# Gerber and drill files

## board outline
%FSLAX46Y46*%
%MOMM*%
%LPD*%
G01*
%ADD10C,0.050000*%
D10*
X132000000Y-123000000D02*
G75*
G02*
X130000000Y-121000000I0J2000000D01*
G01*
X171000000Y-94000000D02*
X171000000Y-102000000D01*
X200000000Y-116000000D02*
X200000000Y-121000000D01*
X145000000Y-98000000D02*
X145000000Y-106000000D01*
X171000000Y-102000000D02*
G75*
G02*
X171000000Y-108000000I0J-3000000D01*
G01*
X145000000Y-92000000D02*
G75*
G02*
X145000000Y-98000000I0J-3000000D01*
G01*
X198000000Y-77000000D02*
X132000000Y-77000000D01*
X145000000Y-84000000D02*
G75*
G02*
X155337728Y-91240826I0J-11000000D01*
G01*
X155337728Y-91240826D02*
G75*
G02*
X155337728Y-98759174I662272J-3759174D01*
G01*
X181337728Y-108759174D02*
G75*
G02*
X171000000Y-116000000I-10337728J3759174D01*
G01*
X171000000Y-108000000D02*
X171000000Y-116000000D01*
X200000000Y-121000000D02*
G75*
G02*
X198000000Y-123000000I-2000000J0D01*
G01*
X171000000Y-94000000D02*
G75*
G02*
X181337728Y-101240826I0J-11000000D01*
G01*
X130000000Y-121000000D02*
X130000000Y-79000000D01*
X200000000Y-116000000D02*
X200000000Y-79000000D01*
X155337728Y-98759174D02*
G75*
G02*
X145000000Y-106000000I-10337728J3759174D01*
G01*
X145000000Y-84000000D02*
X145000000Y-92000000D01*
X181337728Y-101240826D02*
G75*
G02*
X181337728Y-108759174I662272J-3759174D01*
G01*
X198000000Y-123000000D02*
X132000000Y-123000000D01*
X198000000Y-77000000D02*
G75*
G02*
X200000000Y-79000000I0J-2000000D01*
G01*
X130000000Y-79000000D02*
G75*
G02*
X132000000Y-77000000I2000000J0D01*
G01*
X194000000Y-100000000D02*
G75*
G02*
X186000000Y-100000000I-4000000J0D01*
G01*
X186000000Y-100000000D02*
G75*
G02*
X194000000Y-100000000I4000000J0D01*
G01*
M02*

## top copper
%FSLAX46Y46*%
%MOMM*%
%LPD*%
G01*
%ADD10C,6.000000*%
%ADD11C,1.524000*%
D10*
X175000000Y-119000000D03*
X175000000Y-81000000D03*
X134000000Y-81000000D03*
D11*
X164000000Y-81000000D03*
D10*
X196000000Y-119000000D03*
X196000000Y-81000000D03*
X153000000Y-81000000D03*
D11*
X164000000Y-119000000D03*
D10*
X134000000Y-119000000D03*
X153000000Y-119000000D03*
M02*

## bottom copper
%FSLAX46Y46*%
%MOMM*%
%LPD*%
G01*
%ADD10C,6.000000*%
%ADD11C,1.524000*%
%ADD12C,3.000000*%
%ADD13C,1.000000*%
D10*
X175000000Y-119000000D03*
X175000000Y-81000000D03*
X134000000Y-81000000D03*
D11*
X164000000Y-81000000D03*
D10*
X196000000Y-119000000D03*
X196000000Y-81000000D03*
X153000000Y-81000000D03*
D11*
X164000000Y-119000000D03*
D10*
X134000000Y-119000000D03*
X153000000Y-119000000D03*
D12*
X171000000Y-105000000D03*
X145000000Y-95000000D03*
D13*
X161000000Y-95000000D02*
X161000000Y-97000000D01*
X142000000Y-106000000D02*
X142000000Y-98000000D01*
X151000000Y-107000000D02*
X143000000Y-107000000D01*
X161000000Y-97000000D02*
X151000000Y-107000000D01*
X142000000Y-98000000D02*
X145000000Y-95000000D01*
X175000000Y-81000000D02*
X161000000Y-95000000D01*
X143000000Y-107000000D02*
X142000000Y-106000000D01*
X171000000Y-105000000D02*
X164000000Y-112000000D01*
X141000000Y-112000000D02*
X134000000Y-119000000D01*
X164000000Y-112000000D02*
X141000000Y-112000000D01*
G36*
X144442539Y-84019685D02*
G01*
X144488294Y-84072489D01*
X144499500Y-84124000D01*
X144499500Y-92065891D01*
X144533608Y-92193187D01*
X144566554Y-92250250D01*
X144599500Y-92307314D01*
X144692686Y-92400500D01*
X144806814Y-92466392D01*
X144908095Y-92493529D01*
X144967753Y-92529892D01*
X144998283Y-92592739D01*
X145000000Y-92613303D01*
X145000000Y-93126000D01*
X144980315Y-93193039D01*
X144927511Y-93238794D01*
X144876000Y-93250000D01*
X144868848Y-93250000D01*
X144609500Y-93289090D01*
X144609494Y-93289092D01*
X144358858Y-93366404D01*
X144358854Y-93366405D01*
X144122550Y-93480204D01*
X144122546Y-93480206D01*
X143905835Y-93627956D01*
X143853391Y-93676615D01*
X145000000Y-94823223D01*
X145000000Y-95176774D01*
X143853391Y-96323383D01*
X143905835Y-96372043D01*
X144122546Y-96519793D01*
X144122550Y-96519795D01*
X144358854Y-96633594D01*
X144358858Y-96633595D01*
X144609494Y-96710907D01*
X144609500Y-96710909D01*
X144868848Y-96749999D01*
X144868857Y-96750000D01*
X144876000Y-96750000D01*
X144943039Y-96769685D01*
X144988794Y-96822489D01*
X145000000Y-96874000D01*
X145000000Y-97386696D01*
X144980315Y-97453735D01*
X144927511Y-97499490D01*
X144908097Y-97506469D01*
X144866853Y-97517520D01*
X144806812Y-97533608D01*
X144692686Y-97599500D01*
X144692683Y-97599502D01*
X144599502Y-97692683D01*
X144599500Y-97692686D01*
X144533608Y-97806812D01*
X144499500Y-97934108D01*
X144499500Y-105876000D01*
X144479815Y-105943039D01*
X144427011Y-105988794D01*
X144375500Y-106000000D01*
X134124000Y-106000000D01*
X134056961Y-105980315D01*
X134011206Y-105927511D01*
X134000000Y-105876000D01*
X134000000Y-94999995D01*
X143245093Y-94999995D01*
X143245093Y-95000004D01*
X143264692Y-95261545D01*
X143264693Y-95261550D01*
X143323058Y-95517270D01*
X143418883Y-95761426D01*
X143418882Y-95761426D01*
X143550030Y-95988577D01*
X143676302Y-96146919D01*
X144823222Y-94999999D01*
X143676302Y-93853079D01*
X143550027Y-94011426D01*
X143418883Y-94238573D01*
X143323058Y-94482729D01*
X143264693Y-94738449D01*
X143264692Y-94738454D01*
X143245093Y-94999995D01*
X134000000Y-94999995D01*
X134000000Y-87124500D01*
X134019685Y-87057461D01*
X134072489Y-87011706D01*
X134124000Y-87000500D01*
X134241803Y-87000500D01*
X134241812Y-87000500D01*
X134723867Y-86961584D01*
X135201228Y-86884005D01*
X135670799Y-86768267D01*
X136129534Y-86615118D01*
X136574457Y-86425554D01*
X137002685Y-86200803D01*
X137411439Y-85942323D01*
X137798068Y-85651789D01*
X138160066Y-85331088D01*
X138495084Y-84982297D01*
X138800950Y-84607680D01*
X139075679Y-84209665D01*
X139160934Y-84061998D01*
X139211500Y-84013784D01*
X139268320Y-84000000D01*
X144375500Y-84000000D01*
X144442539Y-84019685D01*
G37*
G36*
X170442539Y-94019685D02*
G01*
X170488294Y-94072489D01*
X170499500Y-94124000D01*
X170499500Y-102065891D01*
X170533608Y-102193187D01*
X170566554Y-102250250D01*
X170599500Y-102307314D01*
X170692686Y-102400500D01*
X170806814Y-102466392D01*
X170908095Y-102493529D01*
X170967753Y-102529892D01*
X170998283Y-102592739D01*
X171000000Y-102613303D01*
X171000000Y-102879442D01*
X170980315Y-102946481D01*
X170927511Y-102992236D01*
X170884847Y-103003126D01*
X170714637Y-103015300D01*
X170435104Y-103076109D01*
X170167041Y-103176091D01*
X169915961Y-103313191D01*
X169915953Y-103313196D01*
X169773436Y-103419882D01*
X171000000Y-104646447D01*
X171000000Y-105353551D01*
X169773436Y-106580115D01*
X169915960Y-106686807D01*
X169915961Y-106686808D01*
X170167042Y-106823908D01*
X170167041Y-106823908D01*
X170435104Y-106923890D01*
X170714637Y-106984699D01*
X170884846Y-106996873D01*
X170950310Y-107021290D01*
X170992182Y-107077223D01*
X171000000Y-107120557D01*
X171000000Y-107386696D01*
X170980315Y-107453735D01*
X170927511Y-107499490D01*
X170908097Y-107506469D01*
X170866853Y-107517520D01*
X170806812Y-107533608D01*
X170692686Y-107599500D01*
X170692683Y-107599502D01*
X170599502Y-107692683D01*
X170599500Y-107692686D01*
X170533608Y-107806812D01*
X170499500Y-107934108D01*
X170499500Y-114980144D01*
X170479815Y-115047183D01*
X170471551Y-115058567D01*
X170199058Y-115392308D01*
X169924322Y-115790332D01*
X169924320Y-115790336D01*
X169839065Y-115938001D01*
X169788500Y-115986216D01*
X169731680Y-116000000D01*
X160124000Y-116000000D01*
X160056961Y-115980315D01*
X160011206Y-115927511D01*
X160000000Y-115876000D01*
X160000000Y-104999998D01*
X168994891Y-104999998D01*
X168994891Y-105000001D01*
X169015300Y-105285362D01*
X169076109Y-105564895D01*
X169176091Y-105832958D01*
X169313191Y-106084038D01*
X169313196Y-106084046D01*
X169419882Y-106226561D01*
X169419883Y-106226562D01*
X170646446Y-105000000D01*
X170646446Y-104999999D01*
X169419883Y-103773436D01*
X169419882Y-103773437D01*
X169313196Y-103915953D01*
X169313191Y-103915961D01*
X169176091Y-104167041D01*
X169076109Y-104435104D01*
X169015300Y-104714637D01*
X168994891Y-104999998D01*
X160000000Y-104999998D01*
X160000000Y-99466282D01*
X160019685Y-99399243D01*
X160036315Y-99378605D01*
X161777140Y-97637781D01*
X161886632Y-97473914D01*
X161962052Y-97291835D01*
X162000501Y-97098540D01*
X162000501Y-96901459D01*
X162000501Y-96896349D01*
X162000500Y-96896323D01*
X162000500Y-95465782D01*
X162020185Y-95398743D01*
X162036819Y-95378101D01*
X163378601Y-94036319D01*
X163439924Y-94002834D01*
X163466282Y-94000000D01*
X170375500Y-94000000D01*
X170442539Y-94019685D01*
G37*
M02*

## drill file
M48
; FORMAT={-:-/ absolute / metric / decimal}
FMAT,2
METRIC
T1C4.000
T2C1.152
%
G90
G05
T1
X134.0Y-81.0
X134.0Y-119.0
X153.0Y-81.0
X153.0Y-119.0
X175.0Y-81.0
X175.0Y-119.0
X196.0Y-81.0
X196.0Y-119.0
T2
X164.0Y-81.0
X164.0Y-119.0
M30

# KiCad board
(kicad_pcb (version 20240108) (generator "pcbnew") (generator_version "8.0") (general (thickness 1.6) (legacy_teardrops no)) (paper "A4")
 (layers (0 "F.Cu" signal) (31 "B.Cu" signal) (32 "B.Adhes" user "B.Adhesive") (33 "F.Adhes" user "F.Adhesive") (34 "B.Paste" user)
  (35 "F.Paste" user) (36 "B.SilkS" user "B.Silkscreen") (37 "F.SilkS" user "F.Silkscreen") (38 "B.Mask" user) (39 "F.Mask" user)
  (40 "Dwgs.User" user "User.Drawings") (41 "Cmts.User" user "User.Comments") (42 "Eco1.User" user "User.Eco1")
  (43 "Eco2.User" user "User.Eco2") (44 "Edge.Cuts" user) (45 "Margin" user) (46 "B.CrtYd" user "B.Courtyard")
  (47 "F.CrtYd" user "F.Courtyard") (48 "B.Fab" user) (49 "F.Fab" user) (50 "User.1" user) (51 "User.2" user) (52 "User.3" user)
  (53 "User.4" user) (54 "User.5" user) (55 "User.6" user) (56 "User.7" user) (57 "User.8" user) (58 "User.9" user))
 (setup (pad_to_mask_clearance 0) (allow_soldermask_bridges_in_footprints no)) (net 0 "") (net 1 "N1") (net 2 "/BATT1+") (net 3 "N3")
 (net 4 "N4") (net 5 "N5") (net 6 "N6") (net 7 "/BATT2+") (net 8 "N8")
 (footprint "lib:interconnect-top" (layer "F.Cu") (at 175 119)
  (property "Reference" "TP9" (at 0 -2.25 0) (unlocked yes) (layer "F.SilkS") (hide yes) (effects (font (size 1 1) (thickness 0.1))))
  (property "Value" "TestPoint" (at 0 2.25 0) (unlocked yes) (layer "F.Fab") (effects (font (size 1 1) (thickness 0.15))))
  (pad "1" thru_hole circle (at 0 0) (size 6 6) (drill 4) (layers "*.Cu" "*.Mask") (remove_unused_layers no) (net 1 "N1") (clearance 3)))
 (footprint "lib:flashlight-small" (layer "F.Cu") (at 193 110 0.13)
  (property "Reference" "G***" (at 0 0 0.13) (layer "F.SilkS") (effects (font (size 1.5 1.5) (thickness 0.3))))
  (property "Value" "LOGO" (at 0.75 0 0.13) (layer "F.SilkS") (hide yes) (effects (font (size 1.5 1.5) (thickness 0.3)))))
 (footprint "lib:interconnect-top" (layer "F.Cu") (at 175 81)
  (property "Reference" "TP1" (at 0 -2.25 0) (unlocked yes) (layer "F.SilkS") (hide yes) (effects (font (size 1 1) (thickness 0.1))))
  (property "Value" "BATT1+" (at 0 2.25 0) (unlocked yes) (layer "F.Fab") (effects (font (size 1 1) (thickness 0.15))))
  (pad "1" thru_hole circle (at 0 0) (size 6 6) (drill 4) (layers "*.Cu" "*.Mask") (remove_unused_layers no) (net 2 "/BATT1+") (clearance 3)))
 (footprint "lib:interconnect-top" (layer "F.Cu") (at 134 81)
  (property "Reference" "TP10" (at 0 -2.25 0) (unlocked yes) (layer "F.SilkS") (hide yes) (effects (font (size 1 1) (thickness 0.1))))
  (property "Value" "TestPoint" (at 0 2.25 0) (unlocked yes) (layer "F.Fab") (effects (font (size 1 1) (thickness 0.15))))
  (pad "1" thru_hole circle (at 0 0) (size 6 6) (drill 4) (layers "*.Cu" "*.Mask") (remove_unused_layers no) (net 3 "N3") (clearance 3)))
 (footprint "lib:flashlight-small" (layer "F.Cu") (at 193 90 0.13)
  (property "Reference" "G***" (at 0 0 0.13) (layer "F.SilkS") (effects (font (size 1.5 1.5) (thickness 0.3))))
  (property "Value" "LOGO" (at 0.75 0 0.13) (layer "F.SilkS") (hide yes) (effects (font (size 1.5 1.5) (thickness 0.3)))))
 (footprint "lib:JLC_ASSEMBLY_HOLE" (layer "F.Cu") (at 164 81)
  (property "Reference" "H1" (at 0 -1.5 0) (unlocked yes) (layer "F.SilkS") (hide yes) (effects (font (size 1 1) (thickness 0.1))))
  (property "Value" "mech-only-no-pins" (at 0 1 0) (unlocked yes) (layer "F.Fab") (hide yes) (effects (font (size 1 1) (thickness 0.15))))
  (pad "" np_thru_hole circle (at 0 0) (size 1.524 1.524) (drill 1.152) (layers "F&B.Cu" "*.Mask")))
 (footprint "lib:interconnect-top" (layer "F.Cu") (at 196 119)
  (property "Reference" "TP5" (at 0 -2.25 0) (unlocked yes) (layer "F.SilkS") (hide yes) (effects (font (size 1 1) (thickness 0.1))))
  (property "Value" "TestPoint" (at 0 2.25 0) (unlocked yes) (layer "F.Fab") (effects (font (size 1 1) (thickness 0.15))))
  (pad "1" thru_hole circle (at 0 0) (size 6 6) (drill 4) (layers "*.Cu" "*.Mask") (remove_unused_layers no) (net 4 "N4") (clearance 3)))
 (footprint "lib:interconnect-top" (layer "F.Cu") (at 196 81)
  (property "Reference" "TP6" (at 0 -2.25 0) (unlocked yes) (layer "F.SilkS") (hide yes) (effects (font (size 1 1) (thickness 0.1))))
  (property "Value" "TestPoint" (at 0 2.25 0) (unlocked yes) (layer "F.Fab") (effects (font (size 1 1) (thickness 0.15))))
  (pad "1" thru_hole circle (at 0 0) (size 6 6) (drill 4) (layers "*.Cu" "*.Mask") (remove_unused_layers no) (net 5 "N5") (clearance 3)))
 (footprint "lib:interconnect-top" (layer "F.Cu") (at 153 81)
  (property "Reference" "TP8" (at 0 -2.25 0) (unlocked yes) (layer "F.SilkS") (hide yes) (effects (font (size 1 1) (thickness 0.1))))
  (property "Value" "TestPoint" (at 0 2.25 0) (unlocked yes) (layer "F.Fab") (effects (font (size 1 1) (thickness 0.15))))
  (pad "1" thru_hole circle (at 0 0) (size 6 6) (drill 4) (layers "*.Cu" "*.Mask") (remove_unused_layers no) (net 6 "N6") (clearance 3)))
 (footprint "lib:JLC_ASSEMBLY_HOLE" (layer "F.Cu") (at 164 119)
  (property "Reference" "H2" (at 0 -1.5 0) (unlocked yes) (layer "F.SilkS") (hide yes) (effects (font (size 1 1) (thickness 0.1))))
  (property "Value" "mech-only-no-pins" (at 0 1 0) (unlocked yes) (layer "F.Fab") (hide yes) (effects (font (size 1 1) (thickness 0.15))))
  (pad "" np_thru_hole circle (at 0 0) (size 1.524 1.524) (drill 1.152) (layers "F&B.Cu" "*.Mask")))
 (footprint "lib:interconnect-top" (layer "F.Cu") (at 134 119)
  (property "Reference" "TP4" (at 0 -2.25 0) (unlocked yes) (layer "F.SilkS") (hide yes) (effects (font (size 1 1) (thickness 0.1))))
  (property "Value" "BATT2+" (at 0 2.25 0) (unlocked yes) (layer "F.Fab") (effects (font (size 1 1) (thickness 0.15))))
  (pad "1" thru_hole circle (at 0 0) (size 6 6) (drill 4) (layers "*.Cu" "*.Mask") (remove_unused_layers no) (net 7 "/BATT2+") (clearance 3)))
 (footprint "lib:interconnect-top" (layer "F.Cu") (at 153 119)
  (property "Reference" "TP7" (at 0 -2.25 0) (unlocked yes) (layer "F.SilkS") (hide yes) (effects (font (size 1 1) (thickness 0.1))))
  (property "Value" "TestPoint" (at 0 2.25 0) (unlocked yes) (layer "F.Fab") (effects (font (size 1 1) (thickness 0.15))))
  (pad "1" thru_hole circle (at 0 0) (size 6 6) (drill 4) (layers "*.Cu" "*.Mask") (remove_unused_layers no) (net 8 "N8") (clearance 3)))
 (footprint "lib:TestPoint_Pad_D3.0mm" (layer "B.Cu") (at 171 105 180)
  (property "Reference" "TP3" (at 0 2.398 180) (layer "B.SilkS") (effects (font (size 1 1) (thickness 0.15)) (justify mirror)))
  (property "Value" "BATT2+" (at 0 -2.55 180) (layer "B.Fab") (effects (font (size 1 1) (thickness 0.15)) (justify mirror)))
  (pad "1" smd circle (at 0 0 180) (size 3 3) (layers "B.Cu" "B.Mask") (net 7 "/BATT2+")))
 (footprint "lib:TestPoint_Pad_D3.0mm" (layer "B.Cu") (at 145 95 180)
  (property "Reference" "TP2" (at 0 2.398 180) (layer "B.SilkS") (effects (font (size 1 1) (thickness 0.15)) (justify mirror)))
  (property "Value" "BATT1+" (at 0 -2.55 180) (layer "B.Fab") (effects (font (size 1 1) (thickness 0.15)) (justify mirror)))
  (pad "1" smd circle (at 0 0 180) (size 3 3) (layers "B.Cu" "B.Mask") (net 2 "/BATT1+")))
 (gr_arc (start 132 123) (mid 130.585786 122.414214) (end 130 121) (stroke (width 0.05) (type default)) (layer "Edge.Cuts"))
 (gr_line (start 171 94) (end 171 102) (stroke (width 0.05) (type default)) (layer "Edge.Cuts"))
 (gr_line (start 200 116) (end 200 121) (stroke (width 0.05) (type default)) (layer "Edge.Cuts"))
 (gr_line (start 145 98) (end 145 106) (stroke (width 0.05) (type default)) (layer "Edge.Cuts"))
 (gr_arc (start 171 102) (mid 174 105) (end 171 108) (stroke (width 0.05) (type default)) (layer "Edge.Cuts"))
 (gr_arc (start 145 92) (mid 148 95) (end 145 98) (stroke (width 0.05) (type default)) (layer "Edge.Cuts"))
 (gr_line (start 198 77) (end 132 77) (stroke (width 0.05) (type default)) (layer "Edge.Cuts"))
 (gr_arc (start 145 84) (mid 151.310669 85.990258) (end 155.337728 91.240826) (stroke (width 0.05) (type default)) (layer "Edge.Cuts"))
 (gr_arc (start 155.337728 91.240826) (mid 159.817066 95) (end 155.337728 98.759174) (stroke (width 0.05) (type default))
  (layer "Edge.Cuts"))
 (gr_arc (start 181.337728 108.759174) (mid 177.310669 114.009742) (end 171 116) (stroke (width 0.05) (type default)) (layer "Edge.Cuts"))
 (gr_line (start 171 108) (end 171 116) (stroke (width 0.05) (type default)) (layer "Edge.Cuts"))
 (gr_arc (start 200 121) (mid 199.414214 122.414214) (end 198 123) (stroke (width 0.05) (type default)) (layer "Edge.Cuts"))
 (gr_arc (start 171 94) (mid 177.310669 95.990258) (end 181.337728 101.240826) (stroke (width 0.05) (type default)) (layer "Edge.Cuts"))
 (gr_line (start 130 121) (end 130 79) (stroke (width 0.05) (type default)) (layer "Edge.Cuts"))
 (gr_line (start 200 116) (end 200 79) (stroke (width 0.05) (type default)) (layer "Edge.Cuts"))
 (gr_arc (start 155.337728 98.759174) (mid 151.310669 104.009742) (end 145 106) (stroke (width 0.05) (type default)) (layer "Edge.Cuts"))
 (gr_line (start 145 84) (end 145 92) (stroke (width 0.05) (type default)) (layer "Edge.Cuts"))
 (gr_arc (start 181.337728 101.240826) (mid 185.817066 105) (end 181.337728 108.759174) (stroke (width 0.05) (type default))
  (layer "Edge.Cuts"))
 (gr_line (start 198 123) (end 132 123) (stroke (width 0.05) (type default)) (layer "Edge.Cuts"))
 (gr_arc (start 198 77) (mid 199.414214 77.585786) (end 200 79) (stroke (width 0.05) (type default)) (layer "Edge.Cuts"))
 (gr_arc (start 130 79) (mid 130.585786 77.585786) (end 132 77) (stroke (width 0.05) (type default)) (layer "Edge.Cuts"))
 (gr_circle (center 190 100) (end 194 100) (stroke (width 0.05) (type default)) (fill none) (layer "Edge.Cuts"))
 (segment (start 161 95) (end 161 97) (width 1) (layer "B.Cu") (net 2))
 (segment (start 142 106) (end 142 98) (width 1) (layer "B.Cu") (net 2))
 (segment (start 151 107) (end 143 107) (width 1) (layer "B.Cu") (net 2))
 (segment (start 161 97) (end 151 107) (width 1) (layer "B.Cu") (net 2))
 (segment (start 142 98) (end 145 95) (width 1) (layer "B.Cu") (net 2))
 (segment (start 175 81) (end 161 95) (width 1) (layer "B.Cu") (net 2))
 (segment (start 143 107) (end 142 106) (width 1) (layer "B.Cu") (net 2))
 (segment (start 171 105) (end 164 112) (width 1) (layer "B.Cu") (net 7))
 (segment (start 141 112) (end 134 119) (width 1) (layer "B.Cu") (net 7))
 (segment (start 164 112) (end 141 112) (width 1) (layer "B.Cu") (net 7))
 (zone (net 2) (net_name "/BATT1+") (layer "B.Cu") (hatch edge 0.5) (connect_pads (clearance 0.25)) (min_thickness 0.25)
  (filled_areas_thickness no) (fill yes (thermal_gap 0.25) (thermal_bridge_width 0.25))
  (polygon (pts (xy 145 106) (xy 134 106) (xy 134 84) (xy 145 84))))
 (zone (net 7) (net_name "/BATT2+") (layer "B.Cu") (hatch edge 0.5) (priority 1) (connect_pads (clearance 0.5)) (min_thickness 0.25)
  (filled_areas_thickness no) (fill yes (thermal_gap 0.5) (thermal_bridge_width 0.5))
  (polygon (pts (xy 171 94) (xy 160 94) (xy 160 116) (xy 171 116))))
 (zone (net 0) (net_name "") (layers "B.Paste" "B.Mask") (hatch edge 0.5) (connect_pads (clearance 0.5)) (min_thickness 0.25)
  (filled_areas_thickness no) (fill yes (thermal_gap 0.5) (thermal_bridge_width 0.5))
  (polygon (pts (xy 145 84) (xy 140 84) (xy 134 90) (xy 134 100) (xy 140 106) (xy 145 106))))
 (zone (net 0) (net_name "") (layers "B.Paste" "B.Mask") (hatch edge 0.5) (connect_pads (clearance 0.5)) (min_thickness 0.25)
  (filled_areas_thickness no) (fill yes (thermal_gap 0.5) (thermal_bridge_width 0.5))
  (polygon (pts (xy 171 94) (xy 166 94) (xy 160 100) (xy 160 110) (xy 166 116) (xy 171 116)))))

